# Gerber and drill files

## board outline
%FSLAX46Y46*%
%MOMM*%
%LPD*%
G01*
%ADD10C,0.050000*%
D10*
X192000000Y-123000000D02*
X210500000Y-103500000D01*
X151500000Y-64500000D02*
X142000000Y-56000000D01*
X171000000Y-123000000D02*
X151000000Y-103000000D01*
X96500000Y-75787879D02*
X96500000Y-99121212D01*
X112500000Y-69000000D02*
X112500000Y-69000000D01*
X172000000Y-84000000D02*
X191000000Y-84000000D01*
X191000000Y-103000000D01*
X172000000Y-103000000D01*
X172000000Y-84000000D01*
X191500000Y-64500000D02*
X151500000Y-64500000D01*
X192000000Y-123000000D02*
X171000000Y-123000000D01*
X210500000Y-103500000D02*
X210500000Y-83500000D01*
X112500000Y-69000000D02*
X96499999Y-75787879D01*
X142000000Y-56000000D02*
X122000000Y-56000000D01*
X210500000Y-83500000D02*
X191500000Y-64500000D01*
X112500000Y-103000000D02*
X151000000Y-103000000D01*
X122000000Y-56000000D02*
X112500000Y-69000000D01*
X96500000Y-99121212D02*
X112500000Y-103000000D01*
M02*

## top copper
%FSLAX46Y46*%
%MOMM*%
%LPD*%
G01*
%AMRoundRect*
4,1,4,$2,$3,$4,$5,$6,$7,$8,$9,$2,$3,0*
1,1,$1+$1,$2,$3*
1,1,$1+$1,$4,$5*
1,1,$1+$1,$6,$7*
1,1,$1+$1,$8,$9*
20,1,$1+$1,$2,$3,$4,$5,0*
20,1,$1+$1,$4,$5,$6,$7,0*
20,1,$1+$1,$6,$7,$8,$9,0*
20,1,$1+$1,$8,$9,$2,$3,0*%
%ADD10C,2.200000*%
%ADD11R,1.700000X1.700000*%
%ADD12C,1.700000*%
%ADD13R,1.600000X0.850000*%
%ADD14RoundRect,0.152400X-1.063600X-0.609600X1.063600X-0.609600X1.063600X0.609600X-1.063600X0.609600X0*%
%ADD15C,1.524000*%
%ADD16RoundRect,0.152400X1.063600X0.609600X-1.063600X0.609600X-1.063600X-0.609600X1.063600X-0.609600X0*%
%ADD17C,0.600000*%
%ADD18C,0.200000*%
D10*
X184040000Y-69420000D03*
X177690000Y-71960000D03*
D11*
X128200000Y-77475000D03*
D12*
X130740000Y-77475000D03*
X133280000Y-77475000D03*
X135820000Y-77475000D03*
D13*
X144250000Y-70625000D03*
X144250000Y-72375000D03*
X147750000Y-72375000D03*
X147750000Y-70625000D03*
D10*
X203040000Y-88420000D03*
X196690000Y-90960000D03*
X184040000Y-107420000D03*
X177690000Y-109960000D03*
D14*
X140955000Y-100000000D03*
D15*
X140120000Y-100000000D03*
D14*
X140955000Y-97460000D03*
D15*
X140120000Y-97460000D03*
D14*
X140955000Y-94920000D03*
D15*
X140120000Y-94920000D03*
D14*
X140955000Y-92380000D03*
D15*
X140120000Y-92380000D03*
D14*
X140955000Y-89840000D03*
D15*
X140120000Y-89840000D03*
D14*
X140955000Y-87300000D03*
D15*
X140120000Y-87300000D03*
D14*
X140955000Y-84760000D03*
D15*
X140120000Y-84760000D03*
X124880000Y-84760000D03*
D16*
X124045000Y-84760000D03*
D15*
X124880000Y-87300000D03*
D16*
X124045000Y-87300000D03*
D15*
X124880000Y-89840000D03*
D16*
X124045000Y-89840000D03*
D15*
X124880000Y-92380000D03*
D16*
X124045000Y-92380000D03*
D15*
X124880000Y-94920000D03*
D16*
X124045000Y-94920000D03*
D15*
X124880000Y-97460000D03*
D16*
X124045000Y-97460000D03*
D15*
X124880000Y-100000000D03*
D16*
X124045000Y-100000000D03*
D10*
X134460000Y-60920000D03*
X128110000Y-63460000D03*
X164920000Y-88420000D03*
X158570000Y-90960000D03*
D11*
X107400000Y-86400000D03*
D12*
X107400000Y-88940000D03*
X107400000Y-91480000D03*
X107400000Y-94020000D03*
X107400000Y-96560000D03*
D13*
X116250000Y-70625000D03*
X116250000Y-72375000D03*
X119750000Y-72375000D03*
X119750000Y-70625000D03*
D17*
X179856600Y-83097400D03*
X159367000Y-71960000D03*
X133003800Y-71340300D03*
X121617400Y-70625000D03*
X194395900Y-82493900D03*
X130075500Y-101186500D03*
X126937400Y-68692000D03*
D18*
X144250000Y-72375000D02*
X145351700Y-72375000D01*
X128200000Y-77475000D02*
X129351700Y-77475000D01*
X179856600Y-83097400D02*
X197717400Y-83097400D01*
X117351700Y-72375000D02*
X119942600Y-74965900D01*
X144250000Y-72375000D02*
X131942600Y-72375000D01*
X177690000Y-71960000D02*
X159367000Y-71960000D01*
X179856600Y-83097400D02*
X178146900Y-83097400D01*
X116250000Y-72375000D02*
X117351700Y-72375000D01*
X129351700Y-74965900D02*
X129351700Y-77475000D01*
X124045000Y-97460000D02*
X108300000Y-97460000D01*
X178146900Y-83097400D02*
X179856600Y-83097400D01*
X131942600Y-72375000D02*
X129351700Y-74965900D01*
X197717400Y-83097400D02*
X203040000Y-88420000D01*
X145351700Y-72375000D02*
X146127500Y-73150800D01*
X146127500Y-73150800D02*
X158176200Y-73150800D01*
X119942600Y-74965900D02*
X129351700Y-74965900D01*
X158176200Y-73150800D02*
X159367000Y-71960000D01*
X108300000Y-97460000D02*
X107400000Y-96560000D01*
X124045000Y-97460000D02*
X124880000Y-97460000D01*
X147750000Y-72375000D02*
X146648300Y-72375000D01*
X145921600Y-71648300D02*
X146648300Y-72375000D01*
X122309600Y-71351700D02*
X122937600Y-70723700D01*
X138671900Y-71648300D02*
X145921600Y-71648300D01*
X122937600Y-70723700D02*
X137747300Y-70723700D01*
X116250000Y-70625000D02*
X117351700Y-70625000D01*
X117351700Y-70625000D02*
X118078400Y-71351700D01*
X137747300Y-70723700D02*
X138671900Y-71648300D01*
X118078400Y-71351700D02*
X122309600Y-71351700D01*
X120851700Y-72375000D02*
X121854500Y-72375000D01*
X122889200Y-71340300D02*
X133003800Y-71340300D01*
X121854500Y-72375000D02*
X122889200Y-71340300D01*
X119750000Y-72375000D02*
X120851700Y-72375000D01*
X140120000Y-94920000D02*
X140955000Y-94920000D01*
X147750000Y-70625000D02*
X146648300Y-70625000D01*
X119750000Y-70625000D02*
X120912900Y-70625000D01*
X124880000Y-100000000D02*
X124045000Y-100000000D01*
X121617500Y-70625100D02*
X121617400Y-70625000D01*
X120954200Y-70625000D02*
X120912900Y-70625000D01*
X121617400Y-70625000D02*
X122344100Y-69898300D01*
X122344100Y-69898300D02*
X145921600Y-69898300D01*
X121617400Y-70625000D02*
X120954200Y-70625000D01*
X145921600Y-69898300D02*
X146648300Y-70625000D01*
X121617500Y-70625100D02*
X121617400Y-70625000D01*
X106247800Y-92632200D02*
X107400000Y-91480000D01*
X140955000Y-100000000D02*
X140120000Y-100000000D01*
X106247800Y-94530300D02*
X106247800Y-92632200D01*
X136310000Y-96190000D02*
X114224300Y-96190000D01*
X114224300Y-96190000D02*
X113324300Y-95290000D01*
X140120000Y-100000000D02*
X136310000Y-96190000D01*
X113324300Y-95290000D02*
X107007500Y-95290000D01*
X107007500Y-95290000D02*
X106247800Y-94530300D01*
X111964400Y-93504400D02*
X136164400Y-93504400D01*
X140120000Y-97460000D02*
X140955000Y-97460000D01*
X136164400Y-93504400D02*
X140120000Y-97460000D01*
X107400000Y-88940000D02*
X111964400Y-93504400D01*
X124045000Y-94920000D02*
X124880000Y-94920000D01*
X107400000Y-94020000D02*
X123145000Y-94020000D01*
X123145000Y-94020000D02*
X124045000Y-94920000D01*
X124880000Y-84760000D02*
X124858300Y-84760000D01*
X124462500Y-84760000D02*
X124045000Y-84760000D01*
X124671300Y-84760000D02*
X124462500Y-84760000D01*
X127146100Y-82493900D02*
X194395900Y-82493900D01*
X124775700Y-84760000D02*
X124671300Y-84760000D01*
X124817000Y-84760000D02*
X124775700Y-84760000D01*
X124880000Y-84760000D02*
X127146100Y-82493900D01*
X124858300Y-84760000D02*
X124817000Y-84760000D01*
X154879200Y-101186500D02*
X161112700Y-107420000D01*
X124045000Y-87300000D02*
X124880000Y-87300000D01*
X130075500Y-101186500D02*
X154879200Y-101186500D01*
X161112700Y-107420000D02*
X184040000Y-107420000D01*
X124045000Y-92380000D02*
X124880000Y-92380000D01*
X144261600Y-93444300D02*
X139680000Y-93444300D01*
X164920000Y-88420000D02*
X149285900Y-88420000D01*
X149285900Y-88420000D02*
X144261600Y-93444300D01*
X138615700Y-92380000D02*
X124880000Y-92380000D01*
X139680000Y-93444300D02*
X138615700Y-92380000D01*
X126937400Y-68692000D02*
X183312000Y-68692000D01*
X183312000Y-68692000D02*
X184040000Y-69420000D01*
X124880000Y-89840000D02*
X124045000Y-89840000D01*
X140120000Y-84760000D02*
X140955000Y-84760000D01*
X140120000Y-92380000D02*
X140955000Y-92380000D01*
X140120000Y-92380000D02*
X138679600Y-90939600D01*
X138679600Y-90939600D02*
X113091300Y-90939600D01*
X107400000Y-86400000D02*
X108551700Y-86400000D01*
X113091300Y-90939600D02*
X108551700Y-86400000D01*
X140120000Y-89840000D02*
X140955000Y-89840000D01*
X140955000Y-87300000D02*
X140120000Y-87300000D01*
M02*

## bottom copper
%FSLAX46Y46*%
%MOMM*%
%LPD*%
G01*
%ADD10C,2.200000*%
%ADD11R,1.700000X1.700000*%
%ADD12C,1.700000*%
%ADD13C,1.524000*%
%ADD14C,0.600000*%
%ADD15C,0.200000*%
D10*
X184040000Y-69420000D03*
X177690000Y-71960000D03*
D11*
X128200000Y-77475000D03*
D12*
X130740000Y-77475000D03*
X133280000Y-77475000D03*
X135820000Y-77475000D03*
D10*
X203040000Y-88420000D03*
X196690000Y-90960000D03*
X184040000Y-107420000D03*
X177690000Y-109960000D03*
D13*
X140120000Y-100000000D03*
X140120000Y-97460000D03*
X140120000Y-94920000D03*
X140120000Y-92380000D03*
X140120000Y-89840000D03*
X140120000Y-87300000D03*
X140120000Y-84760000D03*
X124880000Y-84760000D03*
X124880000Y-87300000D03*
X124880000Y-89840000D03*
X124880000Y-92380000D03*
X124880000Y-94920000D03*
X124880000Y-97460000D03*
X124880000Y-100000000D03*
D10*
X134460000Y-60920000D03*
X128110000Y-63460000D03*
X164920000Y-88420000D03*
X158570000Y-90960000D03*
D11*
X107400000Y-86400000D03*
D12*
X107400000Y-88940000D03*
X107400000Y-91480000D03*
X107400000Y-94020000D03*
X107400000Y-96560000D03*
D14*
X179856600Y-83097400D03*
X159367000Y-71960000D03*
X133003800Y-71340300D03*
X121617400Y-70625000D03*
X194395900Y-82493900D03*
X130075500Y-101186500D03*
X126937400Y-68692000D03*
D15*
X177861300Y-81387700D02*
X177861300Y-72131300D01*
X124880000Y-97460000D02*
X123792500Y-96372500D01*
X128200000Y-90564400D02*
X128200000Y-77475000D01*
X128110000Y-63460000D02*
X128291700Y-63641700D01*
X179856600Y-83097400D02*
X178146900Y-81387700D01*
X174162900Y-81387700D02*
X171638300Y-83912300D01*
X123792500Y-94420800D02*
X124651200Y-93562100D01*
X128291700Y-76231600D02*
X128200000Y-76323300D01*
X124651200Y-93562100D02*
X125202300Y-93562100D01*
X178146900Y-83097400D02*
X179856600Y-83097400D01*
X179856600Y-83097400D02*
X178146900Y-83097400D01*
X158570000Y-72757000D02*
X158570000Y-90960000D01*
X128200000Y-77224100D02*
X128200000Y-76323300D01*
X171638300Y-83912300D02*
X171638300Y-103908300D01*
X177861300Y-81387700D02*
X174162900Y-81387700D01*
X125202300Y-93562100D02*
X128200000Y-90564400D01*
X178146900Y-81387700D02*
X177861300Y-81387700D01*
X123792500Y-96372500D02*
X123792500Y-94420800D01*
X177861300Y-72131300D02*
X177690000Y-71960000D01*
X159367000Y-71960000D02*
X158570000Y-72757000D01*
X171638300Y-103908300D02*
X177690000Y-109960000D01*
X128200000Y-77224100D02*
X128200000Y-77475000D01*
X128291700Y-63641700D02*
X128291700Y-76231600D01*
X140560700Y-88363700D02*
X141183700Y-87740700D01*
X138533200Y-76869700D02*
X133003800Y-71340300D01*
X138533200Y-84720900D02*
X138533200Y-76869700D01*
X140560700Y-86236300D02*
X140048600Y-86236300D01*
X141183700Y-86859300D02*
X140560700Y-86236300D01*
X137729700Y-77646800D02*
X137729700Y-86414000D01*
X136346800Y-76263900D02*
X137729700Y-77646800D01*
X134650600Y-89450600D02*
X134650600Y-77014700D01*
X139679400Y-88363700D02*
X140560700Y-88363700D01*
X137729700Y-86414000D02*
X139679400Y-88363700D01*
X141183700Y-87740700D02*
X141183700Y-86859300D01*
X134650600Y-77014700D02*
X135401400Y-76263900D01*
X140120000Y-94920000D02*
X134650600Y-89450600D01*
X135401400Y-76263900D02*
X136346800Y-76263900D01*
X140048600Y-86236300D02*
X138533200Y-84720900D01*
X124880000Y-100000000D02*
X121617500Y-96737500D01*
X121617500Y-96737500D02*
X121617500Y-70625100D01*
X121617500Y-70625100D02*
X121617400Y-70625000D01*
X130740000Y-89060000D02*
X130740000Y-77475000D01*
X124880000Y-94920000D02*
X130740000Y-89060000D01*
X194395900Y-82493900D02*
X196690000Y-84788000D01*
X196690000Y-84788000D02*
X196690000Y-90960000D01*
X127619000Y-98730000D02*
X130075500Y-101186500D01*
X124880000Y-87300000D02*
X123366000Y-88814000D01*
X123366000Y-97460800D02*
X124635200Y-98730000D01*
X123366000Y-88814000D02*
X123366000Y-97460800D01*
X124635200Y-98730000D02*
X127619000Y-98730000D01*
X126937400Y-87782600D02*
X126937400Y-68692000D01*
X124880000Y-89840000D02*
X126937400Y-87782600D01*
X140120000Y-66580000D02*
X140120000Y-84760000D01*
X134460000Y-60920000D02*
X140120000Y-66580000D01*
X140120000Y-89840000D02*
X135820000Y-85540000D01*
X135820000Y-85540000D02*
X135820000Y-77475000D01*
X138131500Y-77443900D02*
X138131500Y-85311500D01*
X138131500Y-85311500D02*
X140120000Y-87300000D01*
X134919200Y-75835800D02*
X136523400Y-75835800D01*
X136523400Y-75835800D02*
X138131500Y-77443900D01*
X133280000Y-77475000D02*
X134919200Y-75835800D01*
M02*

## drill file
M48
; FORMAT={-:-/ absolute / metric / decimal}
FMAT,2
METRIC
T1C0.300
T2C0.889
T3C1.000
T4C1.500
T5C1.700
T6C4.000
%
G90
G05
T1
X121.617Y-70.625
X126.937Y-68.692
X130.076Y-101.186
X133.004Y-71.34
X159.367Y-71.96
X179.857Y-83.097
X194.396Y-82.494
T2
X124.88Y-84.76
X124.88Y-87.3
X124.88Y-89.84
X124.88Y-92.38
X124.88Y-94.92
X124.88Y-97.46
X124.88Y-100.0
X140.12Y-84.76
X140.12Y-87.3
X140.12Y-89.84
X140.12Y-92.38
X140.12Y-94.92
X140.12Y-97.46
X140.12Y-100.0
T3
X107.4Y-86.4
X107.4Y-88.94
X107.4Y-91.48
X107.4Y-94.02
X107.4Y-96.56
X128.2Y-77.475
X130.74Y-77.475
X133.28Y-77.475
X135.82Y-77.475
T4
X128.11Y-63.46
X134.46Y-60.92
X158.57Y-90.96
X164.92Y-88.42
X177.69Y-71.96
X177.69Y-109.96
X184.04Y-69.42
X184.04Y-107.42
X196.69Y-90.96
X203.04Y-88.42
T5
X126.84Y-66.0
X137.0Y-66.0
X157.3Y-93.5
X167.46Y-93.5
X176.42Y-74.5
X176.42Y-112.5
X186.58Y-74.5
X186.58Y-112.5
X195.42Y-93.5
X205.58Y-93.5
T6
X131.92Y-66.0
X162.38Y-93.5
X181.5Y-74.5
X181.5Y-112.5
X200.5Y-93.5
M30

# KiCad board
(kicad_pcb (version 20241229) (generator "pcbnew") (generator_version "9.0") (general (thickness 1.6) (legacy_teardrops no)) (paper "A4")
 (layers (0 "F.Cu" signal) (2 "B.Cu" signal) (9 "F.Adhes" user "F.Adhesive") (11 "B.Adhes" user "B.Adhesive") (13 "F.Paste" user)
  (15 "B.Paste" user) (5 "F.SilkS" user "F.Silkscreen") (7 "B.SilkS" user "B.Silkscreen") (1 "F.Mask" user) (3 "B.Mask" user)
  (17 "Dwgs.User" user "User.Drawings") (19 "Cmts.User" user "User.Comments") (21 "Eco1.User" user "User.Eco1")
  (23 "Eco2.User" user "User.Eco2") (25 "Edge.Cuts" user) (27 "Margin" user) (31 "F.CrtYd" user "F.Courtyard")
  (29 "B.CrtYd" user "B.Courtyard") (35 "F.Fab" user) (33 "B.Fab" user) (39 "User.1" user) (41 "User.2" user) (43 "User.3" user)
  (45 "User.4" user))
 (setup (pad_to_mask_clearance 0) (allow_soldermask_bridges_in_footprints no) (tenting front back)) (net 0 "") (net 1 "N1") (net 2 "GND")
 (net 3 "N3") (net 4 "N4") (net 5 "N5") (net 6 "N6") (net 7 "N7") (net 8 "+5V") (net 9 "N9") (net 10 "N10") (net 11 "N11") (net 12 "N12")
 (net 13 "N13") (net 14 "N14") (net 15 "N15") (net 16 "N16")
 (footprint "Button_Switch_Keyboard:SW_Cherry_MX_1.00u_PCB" (layer "F.Cu") (at 184.04 69.42)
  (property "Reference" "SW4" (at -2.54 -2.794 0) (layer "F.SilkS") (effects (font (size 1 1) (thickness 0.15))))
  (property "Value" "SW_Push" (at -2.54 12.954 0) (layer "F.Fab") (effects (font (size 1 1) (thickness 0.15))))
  (pad "" np_thru_hole circle (at -7.62 5.08) (size 1.7 1.7) (drill 1.7) (layers "*.Cu" "*.Mask"))
  (pad "" np_thru_hole circle (at -2.54 5.08) (size 4 4) (drill 4) (layers "*.Cu" "*.Mask"))
  (pad "" np_thru_hole circle (at 2.54 5.08) (size 1.7 1.7) (drill 1.7) (layers "*.Cu" "*.Mask"))
  (pad "1" thru_hole circle (at 0 0) (size 2.2 2.2) (drill 1.5) (layers "*.Cu" "*.Mask") (remove_unused_layers no) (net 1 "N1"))
  (pad "2" thru_hole circle (at -6.35 2.54) (size 2.2 2.2) (drill 1.5) (layers "*.Cu" "*.Mask") (remove_unused_layers no) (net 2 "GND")))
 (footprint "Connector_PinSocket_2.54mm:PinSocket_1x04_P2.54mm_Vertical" (layer "F.Cu") (at 128.2 77.475 90)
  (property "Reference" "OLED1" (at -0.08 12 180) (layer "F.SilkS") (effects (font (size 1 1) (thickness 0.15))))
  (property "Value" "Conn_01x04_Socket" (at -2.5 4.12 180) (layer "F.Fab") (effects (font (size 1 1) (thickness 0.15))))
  (pad "1" thru_hole rect (at 0 0 90) (size 1.7 1.7) (drill 1) (layers "*.Cu" "*.Mask") (remove_unused_layers no) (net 2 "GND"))
  (pad "2" thru_hole circle (at 0 2.54 90) (size 1.7 1.7) (drill 1) (layers "*.Cu" "*.Mask") (remove_unused_layers no) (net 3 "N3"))
  (pad "3" thru_hole circle (at 0 5.08 90) (size 1.7 1.7) (drill 1) (layers "*.Cu" "*.Mask") (remove_unused_layers no) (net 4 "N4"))
  (pad "4" thru_hole circle (at 0 7.62 90) (size 1.7 1.7) (drill 1) (layers "*.Cu" "*.Mask") (remove_unused_layers no) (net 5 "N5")))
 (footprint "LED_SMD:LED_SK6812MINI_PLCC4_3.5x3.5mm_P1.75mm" (layer "F.Cu") (at 146 71.5)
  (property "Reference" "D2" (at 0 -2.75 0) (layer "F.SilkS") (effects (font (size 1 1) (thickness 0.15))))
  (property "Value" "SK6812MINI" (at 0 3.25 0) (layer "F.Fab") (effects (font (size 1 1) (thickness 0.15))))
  (pad "1" smd rect (at -1.75 -0.875) (size 1.6 0.85) (layers "F.Cu" "F.Mask" "F.Paste") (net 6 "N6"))
  (pad "2" smd rect (at -1.75 0.875) (size 1.6 0.85) (layers "F.Cu" "F.Mask" "F.Paste") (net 2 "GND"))
  (pad "3" smd rect (at 1.75 0.875) (size 1.6 0.85) (layers "F.Cu" "F.Mask" "F.Paste") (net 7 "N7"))
  (pad "4" smd rect (at 1.75 -0.875) (size 1.6 0.85) (layers "F.Cu" "F.Mask" "F.Paste") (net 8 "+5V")))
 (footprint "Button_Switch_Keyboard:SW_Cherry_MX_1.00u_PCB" (layer "F.Cu") (at 203.04 88.42)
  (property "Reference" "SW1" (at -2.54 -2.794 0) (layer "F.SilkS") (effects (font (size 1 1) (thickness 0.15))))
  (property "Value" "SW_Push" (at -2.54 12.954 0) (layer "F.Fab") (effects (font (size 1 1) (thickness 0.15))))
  (pad "" np_thru_hole circle (at -7.62 5.08) (size 1.7 1.7) (drill 1.7) (layers "*.Cu" "*.Mask"))
  (pad "" np_thru_hole circle (at -2.54 5.08) (size 4 4) (drill 4) (layers "*.Cu" "*.Mask"))
  (pad "" np_thru_hole circle (at 2.54 5.08) (size 1.7 1.7) (drill 1.7) (layers "*.Cu" "*.Mask"))
  (pad "1" thru_hole circle (at 0 0) (size 2.2 2.2) (drill 1.5) (layers "*.Cu" "*.Mask") (remove_unused_layers no) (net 2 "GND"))
  (pad "2" thru_hole circle (at -6.35 2.54) (size 2.2 2.2) (drill 1.5) (layers "*.Cu" "*.Mask") (remove_unused_layers no) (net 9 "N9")))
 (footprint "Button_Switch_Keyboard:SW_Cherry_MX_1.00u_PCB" (layer "F.Cu") (at 184.04 107.42)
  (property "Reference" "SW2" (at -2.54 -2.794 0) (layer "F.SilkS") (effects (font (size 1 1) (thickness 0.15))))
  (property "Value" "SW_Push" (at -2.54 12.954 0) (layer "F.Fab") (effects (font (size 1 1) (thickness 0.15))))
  (pad "" np_thru_hole circle (at -7.62 5.08) (size 1.7 1.7) (drill 1.7) (layers "*.Cu" "*.Mask"))
  (pad "" np_thru_hole circle (at -2.54 5.08) (size 4 4) (drill 4) (layers "*.Cu" "*.Mask"))
  (pad "" np_thru_hole circle (at 2.54 5.08) (size 1.7 1.7) (drill 1.7) (layers "*.Cu" "*.Mask"))
  (pad "1" thru_hole circle (at 0 0) (size 2.2 2.2) (drill 1.5) (layers "*.Cu" "*.Mask") (remove_unused_layers no) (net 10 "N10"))
  (pad "2" thru_hole circle (at -6.35 2.54) (size 2.2 2.2) (drill 1.5) (layers "*.Cu" "*.Mask") (remove_unused_layers no) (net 2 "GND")))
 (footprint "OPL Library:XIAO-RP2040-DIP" (layer "F.Cu") (at 132.5 92.38 180)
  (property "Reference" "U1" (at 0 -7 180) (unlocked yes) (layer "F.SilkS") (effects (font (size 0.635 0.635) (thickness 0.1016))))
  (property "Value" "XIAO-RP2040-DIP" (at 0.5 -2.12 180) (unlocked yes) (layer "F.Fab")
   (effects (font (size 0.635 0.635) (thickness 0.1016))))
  (pad "1" smd roundrect (at -8.455 -7.62) (size 2.432 1.524) (layers "F.Cu" "F.Mask") (roundrect_rratio 0.1) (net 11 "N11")
   (thermal_bridge_angle 45))
  (pad "1" thru_hole circle (at -7.62 -7.62) (size 1.524 1.524) (drill 0.889) (layers "*.Cu" "*.Mask") (remove_unused_layers no)
   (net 11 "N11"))
  (pad "2" smd roundrect (at -8.455 -5.08) (size 2.432 1.524) (layers "F.Cu" "F.Mask") (roundrect_rratio 0.1) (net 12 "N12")
   (thermal_bridge_angle 45))
  (pad "2" thru_hole circle (at -7.62 -5.08) (size 1.524 1.524) (drill 0.889) (layers "*.Cu" "*.Mask") (remove_unused_layers no)
   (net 12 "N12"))
  (pad "3" smd roundrect (at -8.455 -2.54) (size 2.432 1.524) (layers "F.Cu" "F.Mask") (roundrect_rratio 0.1) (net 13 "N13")
   (thermal_bridge_angle 45))
  (pad "3" thru_hole circle (at -7.62 -2.54) (size 1.524 1.524) (drill 0.889) (layers "*.Cu" "*.Mask") (remove_unused_layers no)
   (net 13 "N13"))
  (pad "4" smd roundrect (at -8.455 0) (size 2.432 1.524) (layers "F.Cu" "F.Mask") (roundrect_rratio 0.1) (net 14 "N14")
   (thermal_bridge_angle 45))
  (pad "4" thru_hole circle (at -7.62 0) (size 1.524 1.524) (drill 0.889) (layers "*.Cu" "*.Mask") (remove_unused_layers no) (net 14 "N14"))
  (pad "5" smd roundrect (at -8.455 2.54) (size 2.432 1.524) (layers "F.Cu" "F.Mask") (roundrect_rratio 0.1) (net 5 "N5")
   (thermal_bridge_angle 45))
  (pad "5" thru_hole circle (at -7.62 2.54) (size 1.524 1.524) (drill 0.889) (layers "*.Cu" "*.Mask") (remove_unused_layers no) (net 5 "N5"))
  (pad "6" smd roundrect (at -8.455 5.08) (size 2.432 1.524) (layers "F.Cu" "F.Mask") (roundrect_rratio 0.1) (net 4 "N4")
   (thermal_bridge_angle 45))
  (pad "6" thru_hole circle (at -7.62 5.08) (size 1.524 1.524) (drill 0.889) (layers "*.Cu" "*.Mask") (remove_unused_layers no) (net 4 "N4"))
  (pad "7" smd roundrect (at -8.455 7.62) (size 2.432 1.524) (layers "F.Cu" "F.Mask") (roundrect_rratio 0.1) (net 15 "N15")
   (thermal_bridge_angle 45))
  (pad "7" thru_hole circle (at -7.62 7.62) (size 1.524 1.524) (drill 0.889) (layers "*.Cu" "*.Mask") (remove_unused_layers no)
   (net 15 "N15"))
  (pad "8" thru_hole circle (at 7.62 7.62 180) (size 1.524 1.524) (drill 0.889) (layers "*.Cu" "*.Mask") (remove_unused_layers no)
   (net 9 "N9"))
  (pad "8" smd roundrect (at 8.455 7.62 180) (size 2.432 1.524) (layers "F.Cu" "F.Mask") (roundrect_rratio 0.1) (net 9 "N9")
   (thermal_bridge_angle 45))
  (pad "9" thru_hole circle (at 7.62 5.08 180) (size 1.524 1.524) (drill 0.889) (layers "*.Cu" "*.Mask") (remove_unused_layers no)
   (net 10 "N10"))
  (pad "9" smd roundrect (at 8.455 5.08 180) (size 2.432 1.524) (layers "F.Cu" "F.Mask") (roundrect_rratio 0.1) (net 10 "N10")
   (thermal_bridge_angle 45))
  (pad "10" thru_hole circle (at 7.62 2.54 180) (size 1.524 1.524) (drill 0.889) (layers "*.Cu" "*.Mask") (remove_unused_layers no)
   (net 1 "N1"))
  (pad "10" smd roundrect (at 8.455 2.54 180) (size 2.432 1.524) (layers "F.Cu" "F.Mask") (roundrect_rratio 0.1) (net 1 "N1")
   (thermal_bridge_angle 45))
  (pad "11" thru_hole circle (at 7.62 0 180) (size 1.524 1.524) (drill 0.889) (layers "*.Cu" "*.Mask") (remove_unused_layers no)
   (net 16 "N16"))
  (pad "11" smd roundrect (at 8.455 0 180) (size 2.432 1.524) (layers "F.Cu" "F.Mask") (roundrect_rratio 0.1) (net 16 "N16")
   (thermal_bridge_angle 45))
  (pad "12" thru_hole circle (at 7.62 -2.54 180) (size 1.524 1.524) (drill 0.889) (layers "*.Cu" "*.Mask") (remove_unused_layers no)
   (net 3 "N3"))
  (pad "12" smd roundrect (at 8.455 -2.54 180) (size 2.432 1.524) (layers "F.Cu" "F.Mask") (roundrect_rratio 0.1) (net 3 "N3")
   (thermal_bridge_angle 45))
  (pad "13" thru_hole circle (at 7.62 -5.08 180) (size 1.524 1.524) (drill 0.889) (layers "*.Cu" "*.Mask") (remove_unused_layers no)
   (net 2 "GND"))
  (pad "13" smd roundrect (at 8.455 -5.08 180) (size 2.432 1.524) (layers "F.Cu" "F.Mask") (roundrect_rratio 0.1) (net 2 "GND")
   (thermal_bridge_angle 45))
  (pad "14" thru_hole circle (at 7.62 -7.62 180) (size 1.524 1.524) (drill 0.889) (layers "*.Cu" "*.Mask") (remove_unused_layers no)
   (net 8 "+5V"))
  (pad "14" smd roundrect (at 8.455 -7.62 180) (size 2.432 1.524) (layers "F.Cu" "F.Mask") (roundrect_rratio 0.1) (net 8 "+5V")
   (thermal_bridge_angle 45)))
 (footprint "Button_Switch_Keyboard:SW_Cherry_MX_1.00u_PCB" (layer "F.Cu") (at 134.46 60.92)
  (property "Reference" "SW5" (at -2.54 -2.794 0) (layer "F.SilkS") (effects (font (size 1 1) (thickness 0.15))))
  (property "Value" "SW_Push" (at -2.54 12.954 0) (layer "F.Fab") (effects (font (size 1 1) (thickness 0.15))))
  (pad "" np_thru_hole circle (at -7.62 5.08) (size 1.7 1.7) (drill 1.7) (layers "*.Cu" "*.Mask"))
  (pad "" np_thru_hole circle (at -2.54 5.08) (size 4 4) (drill 4) (layers "*.Cu" "*.Mask"))
  (pad "" np_thru_hole circle (at 2.54 5.08) (size 1.7 1.7) (drill 1.7) (layers "*.Cu" "*.Mask"))
  (pad "1" thru_hole circle (at 0 0) (size 2.2 2.2) (drill 1.5) (layers "*.Cu" "*.Mask") (remove_unused_layers no) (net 15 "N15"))
  (pad "2" thru_hole circle (at -6.35 2.54) (size 2.2 2.2) (drill 1.5) (layers "*.Cu" "*.Mask") (remove_unused_layers no) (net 2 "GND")))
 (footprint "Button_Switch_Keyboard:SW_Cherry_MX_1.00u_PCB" (layer "F.Cu") (at 164.92 88.42)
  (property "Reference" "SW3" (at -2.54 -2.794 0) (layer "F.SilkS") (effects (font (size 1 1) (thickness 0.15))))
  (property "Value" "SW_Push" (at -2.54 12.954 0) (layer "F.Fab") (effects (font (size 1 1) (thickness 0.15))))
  (pad "" np_thru_hole circle (at -7.62 5.08) (size 1.7 1.7) (drill 1.7) (layers "*.Cu" "*.Mask"))
  (pad "" np_thru_hole circle (at -2.54 5.08) (size 4 4) (drill 4) (layers "*.Cu" "*.Mask"))
  (pad "" np_thru_hole circle (at 2.54 5.08) (size 1.7 1.7) (drill 1.7) (layers "*.Cu" "*.Mask"))
  (pad "1" thru_hole circle (at 0 0) (size 2.2 2.2) (drill 1.5) (layers "*.Cu" "*.Mask") (remove_unused_layers no) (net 16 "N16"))
  (pad "2" thru_hole circle (at -6.35 2.54) (size 2.2 2.2) (drill 1.5) (layers "*.Cu" "*.Mask") (remove_unused_layers no) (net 2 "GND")))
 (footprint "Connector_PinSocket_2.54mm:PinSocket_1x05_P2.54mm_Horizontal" (layer "F.Cu") (at 107.4 86.4)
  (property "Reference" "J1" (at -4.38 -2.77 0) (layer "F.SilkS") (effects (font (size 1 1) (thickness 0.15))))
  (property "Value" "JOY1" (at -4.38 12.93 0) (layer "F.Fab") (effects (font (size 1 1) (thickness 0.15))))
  (pad "1" thru_hole rect (at 0 0) (size 1.7 1.7) (drill 1) (layers "*.Cu" "*.Mask") (remove_unused_layers no) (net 14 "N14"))
  (pad "2" thru_hole circle (at 0 2.54) (size 1.7 1.7) (drill 1) (layers "*.Cu" "*.Mask") (remove_unused_layers no) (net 12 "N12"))
  (pad "3" thru_hole circle (at 0 5.08) (size 1.7 1.7) (drill 1) (layers "*.Cu" "*.Mask") (remove_unused_layers no) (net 11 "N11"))
  (pad "4" thru_hole circle (at 0 7.62) (size 1.7 1.7) (drill 1) (layers "*.Cu" "*.Mask") (remove_unused_layers no) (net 3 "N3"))
  (pad "5" thru_hole circle (at 0 10.16) (size 1.7 1.7) (drill 1) (layers "*.Cu" "*.Mask") (remove_unused_layers no) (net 2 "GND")))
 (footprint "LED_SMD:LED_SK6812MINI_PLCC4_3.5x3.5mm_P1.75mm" (layer "F.Cu") (at 118 71.5)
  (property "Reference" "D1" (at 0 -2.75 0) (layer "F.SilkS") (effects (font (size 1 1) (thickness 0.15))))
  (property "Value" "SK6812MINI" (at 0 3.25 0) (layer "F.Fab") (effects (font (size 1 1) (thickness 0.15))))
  (pad "1" smd rect (at -1.75 -0.875) (size 1.6 0.85) (layers "F.Cu" "F.Mask" "F.Paste") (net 7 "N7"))
  (pad "2" smd rect (at -1.75 0.875) (size 1.6 0.85) (layers "F.Cu" "F.Mask" "F.Paste") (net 2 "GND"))
  (pad "3" smd rect (at 1.75 0.875) (size 1.6 0.85) (layers "F.Cu" "F.Mask" "F.Paste") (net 13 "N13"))
  (pad "4" smd rect (at 1.75 -0.875) (size 1.6 0.85) (layers "F.Cu" "F.Mask" "F.Paste") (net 8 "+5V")))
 (gr_line (start 192 123) (end 210.5 103.5) (stroke (width 0.05) (type default)) (layer "Edge.Cuts"))
 (gr_line (start 151.5 64.5) (end 142 56) (stroke (width 0.05) (type default)) (layer "Edge.Cuts"))
 (gr_line (start 171 123) (end 151 103) (stroke (width 0.05) (type default)) (layer "Edge.Cuts"))
 (gr_line (start 96.5 75.787879) (end 96.5 99.121212) (stroke (width 0.05) (type default)) (layer "Edge.Cuts"))
 (gr_line (start 112.5 69) (end 112.5 69) (stroke (width 0.05) (type default)) (layer "Edge.Cuts"))
 (gr_rect (start 172 84) (end 191 103) (stroke (width 0.05) (type default)) (fill no) (layer "Edge.Cuts"))
 (gr_line (start 191.5 64.5) (end 151.5 64.5) (stroke (width 0.05) (type default)) (layer "Edge.Cuts"))
 (gr_line (start 192 123) (end 171 123) (stroke (width 0.05) (type default)) (layer "Edge.Cuts"))
 (gr_line (start 210.5 103.5) (end 210.5 83.5) (stroke (width 0.05) (type default)) (layer "Edge.Cuts"))
 (gr_line (start 112.5 69) (end 96.499999 75.787879) (stroke (width 0.05) (type default)) (layer "Edge.Cuts"))
 (gr_line (start 142 56) (end 122 56) (stroke (width 0.05) (type default)) (layer "Edge.Cuts"))
 (gr_line (start 210.5 83.5) (end 191.5 64.5) (stroke (width 0.05) (type default)) (layer "Edge.Cuts"))
 (gr_line (start 112.5 103) (end 151 103) (stroke (width 0.05) (type default)) (layer "Edge.Cuts"))
 (gr_line (start 122 56) (end 112.5 69) (stroke (width 0.05) (type default)) (layer "Edge.Cuts"))
 (gr_line (start 96.5 99.121212) (end 112.5 103) (stroke (width 0.05) (type default)) (layer "Edge.Cuts"))
 (segment (start 144.25 72.375) (end 145.3517 72.375) (width 0.2) (layer "F.Cu") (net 2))
 (segment (start 128.2 77.475) (end 129.3517 77.475) (width 0.2) (layer "F.Cu") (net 2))
 (segment (start 179.8566 83.0974) (end 197.7174 83.0974) (width 0.2) (layer "F.Cu") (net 2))
 (segment (start 117.3517 72.375) (end 119.9426 74.9659) (width 0.2) (layer "F.Cu") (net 2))
 (segment (start 144.25 72.375) (end 131.9426 72.375) (width 0.2) (layer "F.Cu") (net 2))
 (segment (start 177.69 71.96) (end 159.367 71.96) (width 0.2) (layer "F.Cu") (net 2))
 (segment (start 179.8566 83.0974) (end 178.1469 83.0974) (width 0.2) (layer "F.Cu") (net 2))
 (segment (start 116.25 72.375) (end 117.3517 72.375) (width 0.2) (layer "F.Cu") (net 2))
 (segment (start 129.3517 74.9659) (end 129.3517 77.475) (width 0.2) (layer "F.Cu") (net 2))
 (segment (start 124.045 97.46) (end 108.3 97.46) (width 0.2) (layer "F.Cu") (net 2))
 (segment (start 178.1469 83.0974) (end 179.8566 83.0974) (width 0.2) (layer "F.Cu") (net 2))
 (segment (start 131.9426 72.375) (end 129.3517 74.9659) (width 0.2) (layer "F.Cu") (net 2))
 (segment (start 197.7174 83.0974) (end 203.04 88.42) (width 0.2) (layer "F.Cu") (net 2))
 (segment (start 145.3517 72.375) (end 146.1275 73.1508) (width 0.2) (layer "F.Cu") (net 2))
 (segment (start 146.1275 73.1508) (end 158.1762 73.1508) (width 0.2) (layer "F.Cu") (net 2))
 (segment (start 119.9426 74.9659) (end 129.3517 74.9659) (width 0.2) (layer "F.Cu") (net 2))
 (segment (start 158.1762 73.1508) (end 159.367 71.96) (width 0.2) (layer "F.Cu") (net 2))
 (segment (start 108.3 97.46) (end 107.4 96.56) (width 0.2) (layer "F.Cu") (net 2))
 (segment (start 124.045 97.46) (end 124.88 97.46) (width 0.2) (layer "F.Cu") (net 2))
 (via (at 179.8566 83.0974) (size 0.6) (drill 0.3) (layers "F.Cu" "B.Cu") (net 2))
 (via (at 159.367 71.96) (size 0.6) (drill 0.3) (layers "F.Cu" "B.Cu") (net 2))
 (segment (start 177.8613 81.3877) (end 177.8613 72.1313) (width 0.2) (layer "B.Cu") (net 2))
 (segment (start 124.88 97.46) (end 123.7925 96.3725) (width 0.2) (layer "B.Cu") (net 2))
 (segment (start 128.2 90.5644) (end 128.2 77.475) (width 0.2) (layer "B.Cu") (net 2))
 (segment (start 128.11 63.46) (end 128.2917 63.6417) (width 0.2) (layer "B.Cu") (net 2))
 (segment (start 179.8566 83.0974) (end 178.1469 81.3877) (width 0.2) (layer "B.Cu") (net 2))
 (segment (start 174.1629 81.3877) (end 171.6383 83.9123) (width 0.2) (layer "B.Cu") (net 2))
 (segment (start 123.7925 94.4208) (end 124.6512 93.5621) (width 0.2) (layer "B.Cu") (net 2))
 (segment (start 128.2917 76.2316) (end 128.2 76.3233) (width 0.2) (layer "B.Cu") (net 2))
 (segment (start 124.6512 93.5621) (end 125.2023 93.5621) (width 0.2) (layer "B.Cu") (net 2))
 (segment (start 178.1469 83.0974) (end 179.8566 83.0974) (width 0.2) (layer "B.Cu") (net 2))
 (segment (start 179.8566 83.0974) (end 178.1469 83.0974) (width 0.2) (layer "B.Cu") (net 2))
 (segment (start 158.57 72.757) (end 158.57 90.96) (width 0.2) (layer "B.Cu") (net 2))
 (segment (start 128.2 77.2241) (end 128.2 76.3233) (width 0.2) (layer "B.Cu") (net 2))
 (segment (start 171.6383 83.9123) (end 171.6383 103.9083) (width 0.2) (layer "B.Cu") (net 2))
 (segment (start 177.8613 81.3877) (end 174.1629 81.3877) (width 0.2) (layer "B.Cu") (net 2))
 (segment (start 125.2023 93.5621) (end 128.2 90.5644) (width 0.2) (layer "B.Cu") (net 2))
 (segment (start 178.1469 81.3877) (end 177.8613 81.3877) (width 0.2) (layer "B.Cu") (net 2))
 (segment (start 123.7925 96.3725) (end 123.7925 94.4208) (width 0.2) (layer "B.Cu") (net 2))
 (segment (start 177.8613 72.1313) (end 177.69 71.96) (width 0.2) (layer "B.Cu") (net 2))
 (segment (start 159.367 71.96) (end 158.57 72.757) (width 0.2) (layer "B.Cu") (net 2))
 (segment (start 171.6383 103.9083) (end 177.69 109.96) (width 0.2) (layer "B.Cu") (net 2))
 (segment (start 128.2 77.2241) (end 128.2 77.475) (width 0.2) (layer "B.Cu") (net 2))
 (segment (start 128.2917 63.6417) (end 128.2917 76.2316) (width 0.2) (layer "B.Cu") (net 2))
 (segment (start 147.75 72.375) (end 146.6483 72.375) (width 0.2) (layer "F.Cu") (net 7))
 (segment (start 145.9216 71.6483) (end 146.6483 72.375) (width 0.2) (layer "F.Cu") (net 7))
 (segment (start 122.3096 71.3517) (end 122.9376 70.7237) (width 0.2) (layer "F.Cu") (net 7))
 (segment (start 138.6719 71.6483) (end 145.9216 71.6483) (width 0.2) (layer "F.Cu") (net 7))
 (segment (start 122.9376 70.7237) (end 137.7473 70.7237) (width 0.2) (layer "F.Cu") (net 7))
 (segment (start 116.25 70.625) (end 117.3517 70.625) (width 0.2) (layer "F.Cu") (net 7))
 (segment (start 117.3517 70.625) (end 118.0784 71.3517) (width 0.2) (layer "F.Cu") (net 7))
 (segment (start 137.7473 70.7237) (end 138.6719 71.6483) (width 0.2) (layer "F.Cu") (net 7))
 (segment (start 118.0784 71.3517) (end 122.3096 71.3517) (width 0.2) (layer "F.Cu") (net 7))
 (segment (start 120.8517 72.375) (end 121.8545 72.375) (width 0.2) (layer "F.Cu") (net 13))
 (segment (start 122.8892 71.3403) (end 133.0038 71.3403) (width 0.2) (layer "F.Cu") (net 13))
 (segment (start 121.8545 72.375) (end 122.8892 71.3403) (width 0.2) (layer "F.Cu") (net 13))
 (segment (start 119.75 72.375) (end 120.8517 72.375) (width 0.2) (layer "F.Cu") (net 13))
 (segment (start 140.12 94.92) (end 140.955 94.92) (width 0.2) (layer "F.Cu") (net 13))
 (via (at 133.0038 71.3403) (size 0.6) (drill 0.3) (layers "F.Cu" "B.Cu") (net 13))
 (segment (start 140.5607 88.3637) (end 141.1837 87.7407) (width 0.2) (layer "B.Cu") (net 13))
 (segment (start 138.5332 76.8697) (end 133.0038 71.3403) (width 0.2) (layer "B.Cu") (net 13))
 (segment (start 138.5332 84.7209) (end 138.5332 76.8697) (width 0.2) (layer "B.Cu") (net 13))
 (segment (start 140.5607 86.2363) (end 140.0486 86.2363) (width 0.2) (layer "B.Cu") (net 13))
 (segment (start 141.1837 86.8593) (end 140.5607 86.2363) (width 0.2) (layer "B.Cu") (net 13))
 (segment (start 137.7297 77.6468) (end 137.7297 86.414) (width 0.2) (layer "B.Cu") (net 13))
 (segment (start 136.3468 76.2639) (end 137.7297 77.6468) (width 0.2) (layer "B.Cu") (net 13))
 (segment (start 134.6506 89.4506) (end 134.6506 77.0147) (width 0.2) (layer "B.Cu") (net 13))
 (segment (start 139.6794 88.3637) (end 140.5607 88.3637) (width 0.2) (layer "B.Cu") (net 13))
 (segment (start 137.7297 86.414) (end 139.6794 88.3637) (width 0.2) (layer "B.Cu") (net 13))
 (segment (start 141.1837 87.7407) (end 141.1837 86.8593) (width 0.2) (layer "B.Cu") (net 13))
 (segment (start 134.6506 77.0147) (end 135.4014 76.2639) (width 0.2) (layer "B.Cu") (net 13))
 (segment (start 140.12 94.92) (end 134.6506 89.4506) (width 0.2) (layer "B.Cu") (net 13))
 (segment (start 135.4014 76.2639) (end 136.3468 76.2639) (width 0.2) (layer "B.Cu") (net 13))
 (segment (start 140.0486 86.2363) (end 138.5332 84.7209) (width 0.2) (layer "B.Cu") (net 13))
 (segment (start 147.75 70.625) (end 146.6483 70.625) (width 0.2) (layer "F.Cu") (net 8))
 (segment (start 119.75 70.625) (end 120.9129 70.625) (width 0.2) (layer "F.Cu") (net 8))
 (segment (start 124.88 100) (end 124.045 100) (width 0.2) (layer "F.Cu") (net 8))
 (segment (start 121.6175 70.6251) (end 121.6174 70.625) (width 0.2) (layer "F.Cu") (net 8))
 (segment (start 120.9542 70.625) (end 120.9129 70.625) (width 0.2) (layer "F.Cu") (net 8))
 (segment (start 121.6174 70.625) (end 122.3441 69.8983) (width 0.2) (layer "F.Cu") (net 8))
 (segment (start 122.3441 69.8983) (end 145.9216 69.8983) (width 0.2) (layer "F.Cu") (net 8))
 (segment (start 121.6174 70.625) (end 120.9542 70.625) (width 0.2) (layer "F.Cu") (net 8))
 (segment (start 145.9216 69.8983) (end 146.6483 70.625) (width 0.2) (layer "F.Cu") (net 8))
 (segment (start 121.6175 70.6251) (end 121.6174 70.625) (width 0.2) (layer "F.Cu") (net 8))
 (via (at 121.6174 70.625) (size 0.6) (drill 0.3) (layers "F.Cu" "B.Cu") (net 8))
 (segment (start 124.88 100) (end 121.6175 96.7375) (width 0.2) (layer "B.Cu") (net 8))
 (segment (start 121.6175 96.7375) (end 121.6175 70.6251) (width 0.2) (layer "B.Cu") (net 8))
 (segment (start 121.6175 70.6251) (end 121.6174 70.625) (width 0.2) (layer "B.Cu") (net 8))
 (segment (start 106.2478 92.6322) (end 107.4 91.48) (width 0.2) (layer "F.Cu") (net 11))
 (segment (start 140.955 100) (end 140.12 100) (width 0.2) (layer "F.Cu") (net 11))
 (segment (start 106.2478 94.5303) (end 106.2478 92.6322) (width 0.2) (layer "F.Cu") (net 11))
 (segment (start 136.31 96.19) (end 114.2243 96.19) (width 0.2) (layer "F.Cu") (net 11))
 (segment (start 114.2243 96.19) (end 113.3243 95.29) (width 0.2) (layer "F.Cu") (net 11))
 (segment (start 140.12 100) (end 136.31 96.19) (width 0.2) (layer "F.Cu") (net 11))
 (segment (start 113.3243 95.29) (end 107.0075 95.29) (width 0.2) (layer "F.Cu") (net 11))
 (segment (start 107.0075 95.29) (end 106.2478 94.5303) (width 0.2) (layer "F.Cu") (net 11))
 (segment (start 111.9644 93.5044) (end 136.1644 93.5044) (width 0.2) (layer "F.Cu") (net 12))
 (segment (start 140.12 97.46) (end 140.955 97.46) (width 0.2) (layer "F.Cu") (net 12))
 (segment (start 136.1644 93.5044) (end 140.12 97.46) (width 0.2) (layer "F.Cu") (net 12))
 (segment (start 107.4 88.94) (end 111.9644 93.5044) (width 0.2) (layer "F.Cu") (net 12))
 (segment (start 124.045 94.92) (end 124.88 94.92) (width 0.2) (layer "F.Cu") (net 3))
 (segment (start 107.4 94.02) (end 123.145 94.02) (width 0.2) (layer "F.Cu") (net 3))
 (segment (start 123.145 94.02) (end 124.045 94.92) (width 0.2) (layer "F.Cu") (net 3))
 (segment (start 130.74 89.06) (end 130.74 77.475) (width 0.2) (layer "B.Cu") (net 3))
 (segment (start 124.88 94.92) (end 130.74 89.06) (width 0.2) (layer "B.Cu") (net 3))
 (segment (start 124.88 84.76) (end 124.8583 84.76) (width 0.2) (layer "F.Cu") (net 9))
 (segment (start 124.4625 84.76) (end 124.045 84.76) (width 0.2) (layer "F.Cu") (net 9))
 (segment (start 124.6713 84.76) (end 124.4625 84.76) (width 0.2) (layer "F.Cu") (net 9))
 (segment (start 127.1461 82.4939) (end 194.3959 82.4939) (width 0.2) (layer "F.Cu") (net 9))
 (segment (start 124.7757 84.76) (end 124.6713 84.76) (width 0.2) (layer "F.Cu") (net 9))
 (segment (start 124.817 84.76) (end 124.7757 84.76) (width 0.2) (layer "F.Cu") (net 9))
 (segment (start 124.88 84.76) (end 127.1461 82.4939) (width 0.2) (layer "F.Cu") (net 9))
 (segment (start 124.8583 84.76) (end 124.817 84.76) (width 0.2) (layer "F.Cu") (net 9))
 (via (at 194.3959 82.4939) (size 0.6) (drill 0.3) (layers "F.Cu" "B.Cu") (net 9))
 (segment (start 194.3959 82.4939) (end 196.69 84.788) (width 0.2) (layer "B.Cu") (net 9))
 (segment (start 196.69 84.788) (end 196.69 90.96) (width 0.2) (layer "B.Cu") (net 9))
 (segment (start 154.8792 101.1865) (end 161.1127 107.42) (width 0.2) (layer "F.Cu") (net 10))
 (segment (start 124.045 87.3) (end 124.88 87.3) (width 0.2) (layer "F.Cu") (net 10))
 (segment (start 130.0755 101.1865) (end 154.8792 101.1865) (width 0.2) (layer "F.Cu") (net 10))
 (segment (start 161.1127 107.42) (end 184.04 107.42) (width 0.2) (layer "F.Cu") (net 10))
 (via (at 130.0755 101.1865) (size 0.6) (drill 0.3) (layers "F.Cu" "B.Cu") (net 10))
 (segment (start 127.619 98.73) (end 130.0755 101.1865) (width 0.2) (layer "B.Cu") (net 10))
 (segment (start 124.88 87.3) (end 123.366 88.814) (width 0.2) (layer "B.Cu") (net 10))
 (segment (start 123.366 97.4608) (end 124.6352 98.73) (width 0.2) (layer "B.Cu") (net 10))
 (segment (start 123.366 88.814) (end 123.366 97.4608) (width 0.2) (layer "B.Cu") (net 10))
 (segment (start 124.6352 98.73) (end 127.619 98.73) (width 0.2) (layer "B.Cu") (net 10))
 (segment (start 124.045 92.38) (end 124.88 92.38) (width 0.2) (layer "F.Cu") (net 16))
 (segment (start 144.2616 93.4443) (end 139.68 93.4443) (width 0.2) (layer "F.Cu") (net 16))
 (segment (start 164.92 88.42) (end 149.2859 88.42) (width 0.2) (layer "F.Cu") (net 16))
 (segment (start 149.2859 88.42) (end 144.2616 93.4443) (width 0.2) (layer "F.Cu") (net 16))
 (segment (start 138.6157 92.38) (end 124.88 92.38) (width 0.2) (layer "F.Cu") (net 16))
 (segment (start 139.68 93.4443) (end 138.6157 92.38) (width 0.2) (layer "F.Cu") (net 16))
 (segment (start 126.9374 68.692) (end 183.312 68.692) (width 0.2) (layer "F.Cu") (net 1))
 (segment (start 183.312 68.692) (end 184.04 69.42) (width 0.2) (layer "F.Cu") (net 1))
 (segment (start 124.88 89.84) (end 124.045 89.84) (width 0.2) (layer "F.Cu") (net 1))
 (via (at 126.9374 68.692) (size 0.6) (drill 0.3) (layers "F.Cu" "B.Cu") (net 1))
 (segment (start 126.9374 87.7826) (end 126.9374 68.692) (width 0.2) (layer "B.Cu") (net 1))
 (segment (start 124.88 89.84) (end 126.9374 87.7826) (width 0.2) (layer "B.Cu") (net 1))
 (segment (start 140.12 84.76) (end 140.955 84.76) (width 0.2) (layer "F.Cu") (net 15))
 (segment (start 140.12 66.58) (end 140.12 84.76) (width 0.2) (layer "B.Cu") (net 15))
 (segment (start 134.46 60.92) (end 140.12 66.58) (width 0.2) (layer "B.Cu") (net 15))
 (segment (start 140.12 92.38) (end 140.955 92.38) (width 0.2) (layer "F.Cu") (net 14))
 (segment (start 140.12 92.38) (end 138.6796 90.9396) (width 0.2) (layer "F.Cu") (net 14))
 (segment (start 138.6796 90.9396) (end 113.0913 90.9396) (width 0.2) (layer "F.Cu") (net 14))
 (segment (start 107.4 86.4) (end 108.5517 86.4) (width 0.2) (layer "F.Cu") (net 14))
 (segment (start 113.0913 90.9396) (end 108.5517 86.4) (width 0.2) (layer "F.Cu") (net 14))
 (segment (start 140.12 89.84) (end 140.955 89.84) (width 0.2) (layer "F.Cu") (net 5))
 (segment (start 140.12 89.84) (end 135.82 85.54) (width 0.2) (layer "B.Cu") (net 5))
 (segment (start 135.82 85.54) (end 135.82 77.475) (width 0.2) (layer "B.Cu") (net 5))
 (segment (start 140.955 87.3) (end 140.12 87.3) (width 0.2) (layer "F.Cu") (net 4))
 (segment (start 138.1315 77.4439) (end 138.1315 85.3115) (width 0.2) (layer "B.Cu") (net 4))
 (segment (start 138.1315 85.3115) (end 140.12 87.3) (width 0.2) (layer "B.Cu") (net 4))
 (segment (start 134.9192 75.8358) (end 136.5234 75.8358) (width 0.2) (layer "B.Cu") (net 4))
 (segment (start 136.5234 75.8358) (end 138.1315 77.4439) (width 0.2) (layer "B.Cu") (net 4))
 (segment (start 133.28 77.475) (end 134.9192 75.8358) (width 0.2) (layer "B.Cu") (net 4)))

